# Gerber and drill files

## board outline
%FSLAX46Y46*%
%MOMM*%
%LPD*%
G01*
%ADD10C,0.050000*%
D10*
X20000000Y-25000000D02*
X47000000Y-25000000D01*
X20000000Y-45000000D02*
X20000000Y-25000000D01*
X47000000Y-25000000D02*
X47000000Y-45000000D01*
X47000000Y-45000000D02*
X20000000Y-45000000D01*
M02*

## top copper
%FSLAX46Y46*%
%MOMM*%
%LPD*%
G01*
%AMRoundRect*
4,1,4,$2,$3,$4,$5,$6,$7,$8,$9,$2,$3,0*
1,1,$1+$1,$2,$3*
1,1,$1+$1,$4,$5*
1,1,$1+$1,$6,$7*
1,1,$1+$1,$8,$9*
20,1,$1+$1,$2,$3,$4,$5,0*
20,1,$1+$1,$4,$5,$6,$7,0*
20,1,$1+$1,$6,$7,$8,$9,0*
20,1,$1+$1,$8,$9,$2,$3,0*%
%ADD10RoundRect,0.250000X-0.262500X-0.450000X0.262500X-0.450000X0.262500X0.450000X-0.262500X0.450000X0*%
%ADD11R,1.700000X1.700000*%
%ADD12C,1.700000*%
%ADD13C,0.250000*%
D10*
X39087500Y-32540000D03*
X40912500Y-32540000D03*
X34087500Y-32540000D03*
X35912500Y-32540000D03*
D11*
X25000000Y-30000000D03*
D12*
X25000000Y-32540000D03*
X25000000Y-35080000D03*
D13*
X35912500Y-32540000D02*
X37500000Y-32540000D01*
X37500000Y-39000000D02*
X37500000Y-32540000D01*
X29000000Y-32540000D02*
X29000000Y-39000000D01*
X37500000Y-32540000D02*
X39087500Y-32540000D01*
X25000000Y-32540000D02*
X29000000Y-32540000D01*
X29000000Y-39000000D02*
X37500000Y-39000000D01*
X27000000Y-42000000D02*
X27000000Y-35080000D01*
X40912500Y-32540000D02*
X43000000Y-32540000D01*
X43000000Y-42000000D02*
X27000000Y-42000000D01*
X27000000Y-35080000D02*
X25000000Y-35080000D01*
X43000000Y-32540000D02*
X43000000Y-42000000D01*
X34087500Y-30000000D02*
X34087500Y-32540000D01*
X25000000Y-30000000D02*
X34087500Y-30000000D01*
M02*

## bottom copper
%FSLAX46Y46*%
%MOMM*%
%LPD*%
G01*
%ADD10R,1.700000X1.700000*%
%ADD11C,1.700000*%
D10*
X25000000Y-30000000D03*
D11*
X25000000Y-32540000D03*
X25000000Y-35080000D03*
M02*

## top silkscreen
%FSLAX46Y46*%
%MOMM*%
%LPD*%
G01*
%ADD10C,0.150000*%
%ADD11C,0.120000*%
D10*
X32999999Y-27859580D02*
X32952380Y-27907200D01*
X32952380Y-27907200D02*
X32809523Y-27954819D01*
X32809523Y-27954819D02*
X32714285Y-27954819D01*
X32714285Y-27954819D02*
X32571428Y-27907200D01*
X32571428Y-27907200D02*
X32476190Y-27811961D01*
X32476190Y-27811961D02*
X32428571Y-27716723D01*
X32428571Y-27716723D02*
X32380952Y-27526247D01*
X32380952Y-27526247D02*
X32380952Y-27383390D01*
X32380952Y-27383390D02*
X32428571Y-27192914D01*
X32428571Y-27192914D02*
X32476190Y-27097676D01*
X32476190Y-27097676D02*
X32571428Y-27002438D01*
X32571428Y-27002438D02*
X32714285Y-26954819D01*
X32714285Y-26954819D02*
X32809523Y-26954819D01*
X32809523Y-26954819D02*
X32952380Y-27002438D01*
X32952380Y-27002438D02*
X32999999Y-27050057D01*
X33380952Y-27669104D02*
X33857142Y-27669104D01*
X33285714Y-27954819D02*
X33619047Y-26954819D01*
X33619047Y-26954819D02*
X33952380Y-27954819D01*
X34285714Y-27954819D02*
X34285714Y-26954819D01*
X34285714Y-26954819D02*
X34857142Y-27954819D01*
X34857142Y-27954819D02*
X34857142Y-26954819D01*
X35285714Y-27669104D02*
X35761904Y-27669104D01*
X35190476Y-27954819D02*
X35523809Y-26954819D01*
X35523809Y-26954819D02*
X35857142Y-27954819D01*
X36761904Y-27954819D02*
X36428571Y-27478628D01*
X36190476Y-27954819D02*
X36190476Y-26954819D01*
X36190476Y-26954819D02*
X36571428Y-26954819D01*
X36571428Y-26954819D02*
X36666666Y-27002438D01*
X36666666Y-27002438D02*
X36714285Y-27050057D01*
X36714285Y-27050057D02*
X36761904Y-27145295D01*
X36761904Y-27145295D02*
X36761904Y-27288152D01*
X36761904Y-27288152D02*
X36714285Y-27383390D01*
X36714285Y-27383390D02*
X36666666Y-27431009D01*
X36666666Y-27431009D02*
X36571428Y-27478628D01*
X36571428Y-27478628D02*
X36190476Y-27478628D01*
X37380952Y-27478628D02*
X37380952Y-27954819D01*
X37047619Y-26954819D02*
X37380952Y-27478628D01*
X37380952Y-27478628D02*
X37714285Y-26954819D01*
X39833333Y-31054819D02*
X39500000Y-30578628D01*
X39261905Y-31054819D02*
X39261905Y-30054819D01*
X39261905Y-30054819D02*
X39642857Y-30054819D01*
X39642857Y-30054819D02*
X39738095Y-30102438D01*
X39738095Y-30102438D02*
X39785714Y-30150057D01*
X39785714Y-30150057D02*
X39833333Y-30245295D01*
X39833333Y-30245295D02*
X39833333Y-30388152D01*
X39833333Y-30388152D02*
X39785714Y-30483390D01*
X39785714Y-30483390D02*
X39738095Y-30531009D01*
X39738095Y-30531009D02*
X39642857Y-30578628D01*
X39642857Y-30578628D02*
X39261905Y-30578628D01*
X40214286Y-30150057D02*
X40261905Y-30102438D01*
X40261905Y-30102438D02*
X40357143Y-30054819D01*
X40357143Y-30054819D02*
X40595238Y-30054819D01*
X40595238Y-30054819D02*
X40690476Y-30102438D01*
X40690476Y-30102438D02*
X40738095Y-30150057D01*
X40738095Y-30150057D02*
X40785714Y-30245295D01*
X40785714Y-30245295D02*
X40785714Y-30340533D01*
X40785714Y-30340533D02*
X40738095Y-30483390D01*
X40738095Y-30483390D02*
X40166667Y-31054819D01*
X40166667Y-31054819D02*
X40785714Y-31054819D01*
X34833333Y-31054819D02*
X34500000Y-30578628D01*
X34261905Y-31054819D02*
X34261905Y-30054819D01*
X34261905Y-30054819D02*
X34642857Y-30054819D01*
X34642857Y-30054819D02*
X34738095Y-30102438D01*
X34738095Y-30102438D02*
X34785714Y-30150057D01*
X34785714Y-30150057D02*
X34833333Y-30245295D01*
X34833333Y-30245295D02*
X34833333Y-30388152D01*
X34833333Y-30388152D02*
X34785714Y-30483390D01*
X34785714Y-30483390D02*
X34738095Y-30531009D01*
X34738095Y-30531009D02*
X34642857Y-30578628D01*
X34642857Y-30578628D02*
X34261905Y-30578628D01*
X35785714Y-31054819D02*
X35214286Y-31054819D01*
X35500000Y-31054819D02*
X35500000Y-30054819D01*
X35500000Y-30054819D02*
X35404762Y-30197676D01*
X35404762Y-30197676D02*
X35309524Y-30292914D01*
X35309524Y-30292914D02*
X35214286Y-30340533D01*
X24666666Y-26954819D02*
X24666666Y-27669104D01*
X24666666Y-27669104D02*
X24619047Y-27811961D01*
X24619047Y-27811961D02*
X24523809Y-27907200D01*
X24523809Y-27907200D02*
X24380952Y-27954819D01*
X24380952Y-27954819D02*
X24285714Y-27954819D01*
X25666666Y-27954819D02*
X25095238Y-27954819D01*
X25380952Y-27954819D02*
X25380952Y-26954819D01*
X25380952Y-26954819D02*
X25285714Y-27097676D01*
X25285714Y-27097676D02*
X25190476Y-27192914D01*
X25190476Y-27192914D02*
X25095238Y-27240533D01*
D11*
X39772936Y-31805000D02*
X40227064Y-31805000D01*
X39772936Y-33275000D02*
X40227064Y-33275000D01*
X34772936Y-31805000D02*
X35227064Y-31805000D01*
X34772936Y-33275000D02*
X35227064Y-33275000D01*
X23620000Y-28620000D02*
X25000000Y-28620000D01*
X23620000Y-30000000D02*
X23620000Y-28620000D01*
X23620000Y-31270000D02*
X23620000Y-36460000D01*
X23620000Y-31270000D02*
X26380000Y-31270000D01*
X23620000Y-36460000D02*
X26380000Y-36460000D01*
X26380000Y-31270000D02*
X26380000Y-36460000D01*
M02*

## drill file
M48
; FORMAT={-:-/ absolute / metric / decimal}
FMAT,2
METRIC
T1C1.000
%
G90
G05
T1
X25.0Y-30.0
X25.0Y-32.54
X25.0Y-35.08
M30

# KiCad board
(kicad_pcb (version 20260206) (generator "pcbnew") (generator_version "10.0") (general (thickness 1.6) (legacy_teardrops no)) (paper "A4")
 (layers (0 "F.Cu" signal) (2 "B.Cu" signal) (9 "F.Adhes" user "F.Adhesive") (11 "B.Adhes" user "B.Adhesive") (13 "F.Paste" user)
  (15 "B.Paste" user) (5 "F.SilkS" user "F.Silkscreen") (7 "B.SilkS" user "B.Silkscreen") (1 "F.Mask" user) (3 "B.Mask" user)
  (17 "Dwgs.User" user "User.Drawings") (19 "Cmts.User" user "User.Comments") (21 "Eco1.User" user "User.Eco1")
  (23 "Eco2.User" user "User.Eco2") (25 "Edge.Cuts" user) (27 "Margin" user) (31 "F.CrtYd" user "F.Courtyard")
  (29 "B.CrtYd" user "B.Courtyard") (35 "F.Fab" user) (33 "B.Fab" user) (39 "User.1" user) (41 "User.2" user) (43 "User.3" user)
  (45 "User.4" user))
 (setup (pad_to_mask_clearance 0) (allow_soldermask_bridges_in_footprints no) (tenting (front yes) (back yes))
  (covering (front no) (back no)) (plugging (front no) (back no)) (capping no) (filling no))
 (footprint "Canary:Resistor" (layer "F.Cu") (at 40 32.54)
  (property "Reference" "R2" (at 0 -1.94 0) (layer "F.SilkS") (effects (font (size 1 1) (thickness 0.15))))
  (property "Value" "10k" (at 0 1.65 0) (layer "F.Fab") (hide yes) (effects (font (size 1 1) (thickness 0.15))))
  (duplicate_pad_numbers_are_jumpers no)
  (fp_line (start -0.227064 -0.735) (end 0.227064 -0.735) (stroke (width 0.12) (type solid)) (layer "F.SilkS"))
  (fp_line (start -0.227064 0.735) (end 0.227064 0.735) (stroke (width 0.12) (type solid)) (layer "F.SilkS"))
  (pad "1" smd roundrect (at -0.9125 0) (size 1.025 1.4) (layers "F.Cu" "F.Mask" "F.Paste") (roundrect_rratio 0.243902) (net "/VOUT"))
  (pad "2" smd roundrect (at 0.9125 0) (size 1.025 1.4) (layers "F.Cu" "F.Mask" "F.Paste") (roundrect_rratio 0.243902) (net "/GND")))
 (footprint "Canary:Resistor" (layer "F.Cu") (at 35 32.54)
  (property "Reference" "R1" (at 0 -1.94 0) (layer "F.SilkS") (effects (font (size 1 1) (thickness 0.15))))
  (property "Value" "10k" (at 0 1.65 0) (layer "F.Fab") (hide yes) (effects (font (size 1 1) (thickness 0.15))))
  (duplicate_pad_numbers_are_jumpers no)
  (fp_line (start -0.227064 -0.735) (end 0.227064 -0.735) (stroke (width 0.12) (type solid)) (layer "F.SilkS"))
  (fp_line (start -0.227064 0.735) (end 0.227064 0.735) (stroke (width 0.12) (type solid)) (layer "F.SilkS"))
  (pad "1" smd roundrect (at -0.9125 0) (size 1.025 1.4) (layers "F.Cu" "F.Mask" "F.Paste") (roundrect_rratio 0.243902) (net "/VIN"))
  (pad "2" smd roundrect (at 0.9125 0) (size 1.025 1.4) (layers "F.Cu" "F.Mask" "F.Paste") (roundrect_rratio 0.243902) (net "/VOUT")))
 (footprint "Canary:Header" (layer "F.Cu") (at 25 30)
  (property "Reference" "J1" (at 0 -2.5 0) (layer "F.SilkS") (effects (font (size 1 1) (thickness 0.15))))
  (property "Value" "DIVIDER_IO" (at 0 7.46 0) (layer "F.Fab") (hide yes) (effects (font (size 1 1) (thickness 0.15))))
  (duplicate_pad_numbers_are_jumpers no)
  (fp_line (start -1.38 -1.38) (end 0 -1.38) (stroke (width 0.12) (type solid)) (layer "F.SilkS"))
  (fp_line (start -1.38 0) (end -1.38 -1.38) (stroke (width 0.12) (type solid)) (layer "F.SilkS"))
  (fp_line (start -1.38 1.27) (end -1.38 6.46) (stroke (width 0.12) (type solid)) (layer "F.SilkS"))
  (fp_line (start -1.38 1.27) (end 1.38 1.27) (stroke (width 0.12) (type solid)) (layer "F.SilkS"))
  (fp_line (start -1.38 6.46) (end 1.38 6.46) (stroke (width 0.12) (type solid)) (layer "F.SilkS"))
  (fp_line (start 1.38 1.27) (end 1.38 6.46) (stroke (width 0.12) (type solid)) (layer "F.SilkS"))
  (pad "1" thru_hole rect (at 0 0) (size 1.7 1.7) (drill 1) (layers "*.Cu" "*.Mask") (remove_unused_layers no) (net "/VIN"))
  (pad "2" thru_hole circle (at 0 2.54) (size 1.7 1.7) (drill 1) (layers "*.Cu" "*.Mask") (remove_unused_layers no) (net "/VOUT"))
  (pad "3" thru_hole circle (at 0 5.08) (size 1.7 1.7) (drill 1) (layers "*.Cu" "*.Mask") (remove_unused_layers no) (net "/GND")))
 (gr_line (start 20 25) (end 47 25) (stroke (width 0.05) (type default)) (layer "Edge.Cuts"))
 (gr_line (start 20 45) (end 20 25) (stroke (width 0.05) (type default)) (layer "Edge.Cuts"))
 (gr_line (start 47 25) (end 47 45) (stroke (width 0.05) (type default)) (layer "Edge.Cuts"))
 (gr_line (start 47 45) (end 20 45) (stroke (width 0.05) (type default)) (layer "Edge.Cuts"))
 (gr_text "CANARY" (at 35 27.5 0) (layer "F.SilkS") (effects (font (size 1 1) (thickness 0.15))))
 (segment (start 35.9125 32.54) (end 37.5 32.54) (width 0.25) (layer "F.Cu") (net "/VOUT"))
 (segment (start 37.5 39) (end 37.5 32.54) (width 0.25) (layer "F.Cu") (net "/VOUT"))
 (segment (start 29 32.54) (end 29 39) (width 0.25) (layer "F.Cu") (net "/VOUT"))
 (segment (start 37.5 32.54) (end 39.0875 32.54) (width 0.25) (layer "F.Cu") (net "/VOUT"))
 (segment (start 25 32.54) (end 29 32.54) (width 0.25) (layer "F.Cu") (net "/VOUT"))
 (segment (start 29 39) (end 37.5 39) (width 0.25) (layer "F.Cu") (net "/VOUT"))
 (segment (start 27 42) (end 27 35.08) (width 0.25) (layer "F.Cu") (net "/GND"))
 (segment (start 40.9125 32.54) (end 43 32.54) (width 0.25) (layer "F.Cu") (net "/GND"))
 (segment (start 43 42) (end 27 42) (width 0.25) (layer "F.Cu") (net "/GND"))
 (segment (start 27 35.08) (end 25 35.08) (width 0.25) (layer "F.Cu") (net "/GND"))
 (segment (start 43 32.54) (end 43 42) (width 0.25) (layer "F.Cu") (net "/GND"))
 (segment (start 34.0875 30) (end 34.0875 32.54) (width 0.25) (layer "F.Cu") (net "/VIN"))
 (segment (start 25 30) (end 34.0875 30) (width 0.25) (layer "F.Cu") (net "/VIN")))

